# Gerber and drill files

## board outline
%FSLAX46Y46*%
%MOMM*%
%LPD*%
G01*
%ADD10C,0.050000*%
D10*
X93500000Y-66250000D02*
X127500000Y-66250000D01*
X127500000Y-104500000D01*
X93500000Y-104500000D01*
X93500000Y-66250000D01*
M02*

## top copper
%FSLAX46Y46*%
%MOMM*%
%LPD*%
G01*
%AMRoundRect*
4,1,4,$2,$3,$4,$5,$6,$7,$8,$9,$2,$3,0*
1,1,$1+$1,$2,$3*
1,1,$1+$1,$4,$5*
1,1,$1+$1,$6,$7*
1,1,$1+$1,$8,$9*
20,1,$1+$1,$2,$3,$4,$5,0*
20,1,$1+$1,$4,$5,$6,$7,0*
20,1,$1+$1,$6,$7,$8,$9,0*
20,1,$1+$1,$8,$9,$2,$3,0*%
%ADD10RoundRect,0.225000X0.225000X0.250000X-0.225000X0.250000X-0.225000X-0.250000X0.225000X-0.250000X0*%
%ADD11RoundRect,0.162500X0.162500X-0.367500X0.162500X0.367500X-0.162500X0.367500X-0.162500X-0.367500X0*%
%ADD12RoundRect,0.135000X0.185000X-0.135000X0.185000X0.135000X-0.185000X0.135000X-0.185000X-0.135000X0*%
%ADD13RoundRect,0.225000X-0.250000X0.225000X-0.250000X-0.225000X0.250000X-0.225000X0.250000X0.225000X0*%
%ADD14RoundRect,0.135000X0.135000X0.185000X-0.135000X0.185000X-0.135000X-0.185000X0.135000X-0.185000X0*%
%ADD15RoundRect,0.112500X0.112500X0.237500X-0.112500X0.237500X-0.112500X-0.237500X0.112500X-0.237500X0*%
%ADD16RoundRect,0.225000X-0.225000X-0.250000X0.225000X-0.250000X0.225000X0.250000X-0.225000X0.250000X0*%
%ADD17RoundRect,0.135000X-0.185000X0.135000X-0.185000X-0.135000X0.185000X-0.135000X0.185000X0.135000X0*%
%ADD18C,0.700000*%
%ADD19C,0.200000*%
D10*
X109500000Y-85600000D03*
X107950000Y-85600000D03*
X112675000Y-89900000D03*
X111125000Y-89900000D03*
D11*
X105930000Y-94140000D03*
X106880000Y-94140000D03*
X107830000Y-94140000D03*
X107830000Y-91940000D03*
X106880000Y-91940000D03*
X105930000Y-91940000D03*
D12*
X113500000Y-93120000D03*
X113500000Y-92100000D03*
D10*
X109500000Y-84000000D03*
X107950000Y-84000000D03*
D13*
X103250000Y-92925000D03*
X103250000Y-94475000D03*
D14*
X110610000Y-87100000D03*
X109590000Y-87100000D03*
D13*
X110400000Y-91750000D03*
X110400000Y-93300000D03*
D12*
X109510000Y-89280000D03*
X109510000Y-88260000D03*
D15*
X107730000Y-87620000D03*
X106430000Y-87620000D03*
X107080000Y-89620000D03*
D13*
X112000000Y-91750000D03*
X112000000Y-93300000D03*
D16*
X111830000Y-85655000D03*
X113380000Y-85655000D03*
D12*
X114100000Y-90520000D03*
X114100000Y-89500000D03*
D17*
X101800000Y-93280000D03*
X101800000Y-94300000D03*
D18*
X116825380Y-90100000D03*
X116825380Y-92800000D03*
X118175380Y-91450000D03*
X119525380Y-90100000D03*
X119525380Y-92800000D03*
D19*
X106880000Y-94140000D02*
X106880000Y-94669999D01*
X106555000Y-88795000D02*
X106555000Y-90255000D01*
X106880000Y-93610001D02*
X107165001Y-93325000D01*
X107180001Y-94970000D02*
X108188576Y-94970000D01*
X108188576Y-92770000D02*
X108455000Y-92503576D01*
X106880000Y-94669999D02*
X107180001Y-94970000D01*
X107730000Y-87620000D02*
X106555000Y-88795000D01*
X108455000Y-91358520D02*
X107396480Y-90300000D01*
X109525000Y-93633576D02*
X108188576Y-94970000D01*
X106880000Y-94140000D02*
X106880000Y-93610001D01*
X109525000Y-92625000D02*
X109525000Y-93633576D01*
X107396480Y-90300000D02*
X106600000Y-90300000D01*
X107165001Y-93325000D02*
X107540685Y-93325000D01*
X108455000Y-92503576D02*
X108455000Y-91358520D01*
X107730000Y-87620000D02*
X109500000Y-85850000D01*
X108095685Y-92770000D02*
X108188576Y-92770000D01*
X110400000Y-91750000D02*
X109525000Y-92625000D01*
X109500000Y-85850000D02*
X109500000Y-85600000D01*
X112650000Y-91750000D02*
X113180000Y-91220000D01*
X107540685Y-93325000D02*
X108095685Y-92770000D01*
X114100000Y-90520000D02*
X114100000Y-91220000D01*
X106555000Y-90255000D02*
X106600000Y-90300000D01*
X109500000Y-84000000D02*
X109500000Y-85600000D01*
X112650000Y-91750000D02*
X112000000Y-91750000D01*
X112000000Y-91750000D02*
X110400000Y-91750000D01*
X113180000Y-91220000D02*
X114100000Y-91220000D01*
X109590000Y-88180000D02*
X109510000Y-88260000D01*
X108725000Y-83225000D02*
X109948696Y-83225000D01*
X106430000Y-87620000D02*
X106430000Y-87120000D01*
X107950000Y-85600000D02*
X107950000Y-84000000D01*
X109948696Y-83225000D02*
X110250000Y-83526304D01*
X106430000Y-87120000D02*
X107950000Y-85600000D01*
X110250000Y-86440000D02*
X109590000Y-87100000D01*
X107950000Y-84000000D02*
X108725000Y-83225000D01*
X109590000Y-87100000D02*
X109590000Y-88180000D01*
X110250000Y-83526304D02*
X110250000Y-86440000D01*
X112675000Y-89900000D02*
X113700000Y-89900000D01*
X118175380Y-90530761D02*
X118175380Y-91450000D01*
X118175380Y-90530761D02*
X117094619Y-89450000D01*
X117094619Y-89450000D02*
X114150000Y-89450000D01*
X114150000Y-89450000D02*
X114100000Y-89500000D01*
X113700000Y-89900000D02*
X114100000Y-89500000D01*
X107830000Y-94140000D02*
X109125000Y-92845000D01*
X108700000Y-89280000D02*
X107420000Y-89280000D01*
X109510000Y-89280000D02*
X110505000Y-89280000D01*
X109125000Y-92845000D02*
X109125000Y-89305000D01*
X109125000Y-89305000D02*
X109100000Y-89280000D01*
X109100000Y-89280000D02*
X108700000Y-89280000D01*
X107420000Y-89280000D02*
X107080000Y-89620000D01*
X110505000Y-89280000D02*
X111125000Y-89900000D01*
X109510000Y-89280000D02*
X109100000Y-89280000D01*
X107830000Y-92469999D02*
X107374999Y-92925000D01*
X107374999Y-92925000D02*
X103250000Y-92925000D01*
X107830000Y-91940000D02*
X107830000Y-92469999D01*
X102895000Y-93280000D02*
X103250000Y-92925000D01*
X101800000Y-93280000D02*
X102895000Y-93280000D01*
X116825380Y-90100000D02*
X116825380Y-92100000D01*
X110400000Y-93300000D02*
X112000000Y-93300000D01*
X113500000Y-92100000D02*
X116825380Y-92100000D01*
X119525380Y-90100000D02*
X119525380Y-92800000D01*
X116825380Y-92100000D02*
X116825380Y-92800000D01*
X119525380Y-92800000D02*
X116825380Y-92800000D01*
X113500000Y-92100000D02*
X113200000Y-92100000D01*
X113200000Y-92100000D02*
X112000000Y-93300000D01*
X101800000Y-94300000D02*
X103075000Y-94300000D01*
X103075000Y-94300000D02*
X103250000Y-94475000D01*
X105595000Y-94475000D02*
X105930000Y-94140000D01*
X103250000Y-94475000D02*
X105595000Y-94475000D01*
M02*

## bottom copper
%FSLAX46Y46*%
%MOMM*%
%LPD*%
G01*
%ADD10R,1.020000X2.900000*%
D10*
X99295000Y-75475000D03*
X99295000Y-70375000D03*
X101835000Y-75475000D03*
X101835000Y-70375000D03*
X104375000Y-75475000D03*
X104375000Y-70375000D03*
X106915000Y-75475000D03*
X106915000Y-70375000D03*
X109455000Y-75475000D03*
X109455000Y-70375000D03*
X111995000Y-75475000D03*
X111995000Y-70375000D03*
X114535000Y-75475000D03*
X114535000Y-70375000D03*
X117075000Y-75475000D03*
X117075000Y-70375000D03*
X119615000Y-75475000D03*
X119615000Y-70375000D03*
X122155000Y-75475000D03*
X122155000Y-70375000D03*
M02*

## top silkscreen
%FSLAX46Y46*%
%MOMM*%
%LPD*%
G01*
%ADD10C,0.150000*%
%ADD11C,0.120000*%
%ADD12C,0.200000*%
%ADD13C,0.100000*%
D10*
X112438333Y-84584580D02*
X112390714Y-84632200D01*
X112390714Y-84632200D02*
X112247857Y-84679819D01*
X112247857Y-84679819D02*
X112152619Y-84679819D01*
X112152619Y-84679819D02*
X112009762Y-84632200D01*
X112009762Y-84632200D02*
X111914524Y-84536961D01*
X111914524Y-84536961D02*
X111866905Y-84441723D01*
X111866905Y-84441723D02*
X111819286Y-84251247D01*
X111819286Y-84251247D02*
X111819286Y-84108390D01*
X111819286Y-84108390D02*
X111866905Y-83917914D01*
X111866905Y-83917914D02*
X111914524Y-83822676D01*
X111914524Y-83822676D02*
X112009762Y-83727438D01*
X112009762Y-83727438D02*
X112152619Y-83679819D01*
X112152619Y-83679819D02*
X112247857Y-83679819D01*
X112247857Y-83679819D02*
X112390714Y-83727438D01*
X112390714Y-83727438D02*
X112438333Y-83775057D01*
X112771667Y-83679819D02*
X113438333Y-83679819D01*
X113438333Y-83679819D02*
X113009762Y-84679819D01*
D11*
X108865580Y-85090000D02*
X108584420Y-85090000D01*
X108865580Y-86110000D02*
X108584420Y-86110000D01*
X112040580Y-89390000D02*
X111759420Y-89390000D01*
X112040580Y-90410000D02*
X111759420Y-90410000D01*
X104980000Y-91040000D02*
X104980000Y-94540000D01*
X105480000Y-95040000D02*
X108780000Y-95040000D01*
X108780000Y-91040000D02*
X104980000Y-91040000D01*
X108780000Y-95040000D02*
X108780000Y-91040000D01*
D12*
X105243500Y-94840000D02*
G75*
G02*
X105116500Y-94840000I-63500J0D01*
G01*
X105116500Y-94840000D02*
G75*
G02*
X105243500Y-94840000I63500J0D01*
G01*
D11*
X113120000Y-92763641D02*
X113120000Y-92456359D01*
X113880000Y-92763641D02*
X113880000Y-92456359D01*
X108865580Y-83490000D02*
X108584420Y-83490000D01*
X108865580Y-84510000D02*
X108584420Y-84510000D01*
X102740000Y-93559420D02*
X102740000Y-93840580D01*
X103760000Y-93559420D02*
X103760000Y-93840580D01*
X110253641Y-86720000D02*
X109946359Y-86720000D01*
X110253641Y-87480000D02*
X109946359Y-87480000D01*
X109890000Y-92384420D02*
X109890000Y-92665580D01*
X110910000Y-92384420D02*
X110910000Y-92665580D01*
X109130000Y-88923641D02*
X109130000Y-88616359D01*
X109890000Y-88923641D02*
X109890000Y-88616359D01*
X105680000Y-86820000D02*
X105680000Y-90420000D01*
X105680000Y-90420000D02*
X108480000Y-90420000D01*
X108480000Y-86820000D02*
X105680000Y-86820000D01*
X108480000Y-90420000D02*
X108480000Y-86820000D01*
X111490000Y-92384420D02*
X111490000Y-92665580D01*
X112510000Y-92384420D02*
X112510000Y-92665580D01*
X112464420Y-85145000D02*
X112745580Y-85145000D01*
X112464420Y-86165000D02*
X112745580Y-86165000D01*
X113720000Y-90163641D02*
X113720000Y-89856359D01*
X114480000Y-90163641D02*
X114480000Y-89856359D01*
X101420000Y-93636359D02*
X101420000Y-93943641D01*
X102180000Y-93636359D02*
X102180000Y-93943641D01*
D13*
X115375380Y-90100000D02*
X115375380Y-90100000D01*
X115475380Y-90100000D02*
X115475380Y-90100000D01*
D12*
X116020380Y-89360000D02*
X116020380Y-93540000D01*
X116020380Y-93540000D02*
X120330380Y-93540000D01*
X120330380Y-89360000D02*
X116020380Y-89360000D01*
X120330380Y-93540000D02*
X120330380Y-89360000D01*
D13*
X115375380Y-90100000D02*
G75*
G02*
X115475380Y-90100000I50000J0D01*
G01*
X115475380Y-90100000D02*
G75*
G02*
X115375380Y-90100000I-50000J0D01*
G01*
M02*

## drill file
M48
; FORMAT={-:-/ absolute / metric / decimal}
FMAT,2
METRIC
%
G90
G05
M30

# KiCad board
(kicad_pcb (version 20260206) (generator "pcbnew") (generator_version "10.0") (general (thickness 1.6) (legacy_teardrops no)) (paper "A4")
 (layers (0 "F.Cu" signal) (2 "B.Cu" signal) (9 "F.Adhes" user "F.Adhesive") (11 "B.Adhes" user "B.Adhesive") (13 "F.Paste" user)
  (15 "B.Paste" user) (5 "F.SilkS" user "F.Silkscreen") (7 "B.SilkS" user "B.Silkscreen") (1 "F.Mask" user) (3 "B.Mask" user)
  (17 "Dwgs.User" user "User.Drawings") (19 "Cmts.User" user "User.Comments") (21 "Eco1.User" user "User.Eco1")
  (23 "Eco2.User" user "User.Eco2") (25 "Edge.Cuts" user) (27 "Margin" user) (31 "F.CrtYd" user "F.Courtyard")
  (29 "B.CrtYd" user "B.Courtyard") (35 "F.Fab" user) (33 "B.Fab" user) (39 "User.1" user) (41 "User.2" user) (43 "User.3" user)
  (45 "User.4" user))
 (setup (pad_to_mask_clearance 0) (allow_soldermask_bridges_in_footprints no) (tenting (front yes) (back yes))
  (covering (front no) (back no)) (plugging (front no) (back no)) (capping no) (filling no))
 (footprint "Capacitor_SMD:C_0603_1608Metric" (layer "F.Cu") (at 108.725 85.6 180)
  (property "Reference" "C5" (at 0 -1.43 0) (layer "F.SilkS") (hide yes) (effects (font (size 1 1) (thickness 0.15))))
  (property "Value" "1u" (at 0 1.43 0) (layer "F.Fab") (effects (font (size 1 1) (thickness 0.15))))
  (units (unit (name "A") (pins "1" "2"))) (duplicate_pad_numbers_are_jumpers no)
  (fp_line (start -0.14058 0.51) (end 0.14058 0.51) (stroke (width 0.12) (type solid)) (layer "F.SilkS"))
  (fp_line (start -0.14058 -0.51) (end 0.14058 -0.51) (stroke (width 0.12) (type solid)) (layer "F.SilkS"))
  (pad "1" smd roundrect (at -0.775 0 180) (size 0.9 0.95) (layers "F.Cu" "F.Mask" "F.Paste") (roundrect_rratio 0.25) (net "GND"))
  (pad "2" smd roundrect (at 0.775 0 180) (size 0.9 0.95) (layers "F.Cu" "F.Mask" "F.Paste") (roundrect_rratio 0.25) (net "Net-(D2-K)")))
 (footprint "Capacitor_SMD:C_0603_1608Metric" (layer "F.Cu") (at 111.9 89.9 180)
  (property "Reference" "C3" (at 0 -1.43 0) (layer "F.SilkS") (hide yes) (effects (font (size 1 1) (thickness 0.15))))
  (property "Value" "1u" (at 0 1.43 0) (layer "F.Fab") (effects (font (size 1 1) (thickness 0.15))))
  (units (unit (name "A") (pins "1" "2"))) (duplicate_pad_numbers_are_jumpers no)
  (fp_line (start -0.14058 0.51) (end 0.14058 0.51) (stroke (width 0.12) (type solid)) (layer "F.SilkS"))
  (fp_line (start -0.14058 -0.51) (end 0.14058 -0.51) (stroke (width 0.12) (type solid)) (layer "F.SilkS"))
  (pad "1" smd roundrect (at -0.775 0 180) (size 0.9 0.95) (layers "F.Cu" "F.Mask" "F.Paste") (roundrect_rratio 0.25) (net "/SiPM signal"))
  (pad "2" smd roundrect (at 0.775 0 180) (size 0.9 0.95) (layers "F.Cu" "F.Mask" "F.Paste") (roundrect_rratio 0.25) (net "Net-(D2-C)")))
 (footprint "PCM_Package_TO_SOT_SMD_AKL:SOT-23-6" (layer "F.Cu") (at 106.88 93.04 90)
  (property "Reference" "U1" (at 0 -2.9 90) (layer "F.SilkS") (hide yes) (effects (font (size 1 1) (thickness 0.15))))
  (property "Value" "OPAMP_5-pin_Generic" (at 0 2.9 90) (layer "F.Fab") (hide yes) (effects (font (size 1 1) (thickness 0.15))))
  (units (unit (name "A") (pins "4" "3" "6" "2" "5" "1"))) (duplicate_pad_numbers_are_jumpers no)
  (fp_line (start 2 -1.9) (end -1.5 -1.9) (stroke (width 0.12) (type solid)) (layer "F.SilkS"))
  (fp_line (start -2 -1.4) (end -2 1.9) (stroke (width 0.12) (type solid)) (layer "F.SilkS"))
  (fp_line (start 2 1.9) (end 2 -1.9) (stroke (width 0.12) (type solid)) (layer "F.SilkS"))
  (fp_line (start -2 1.9) (end 2 1.9) (stroke (width 0.12) (type solid)) (layer "F.SilkS"))
  (fp_circle (center -1.8 -1.7) (end -1.7365 -1.7) (stroke (width 0.2) (type solid)) (fill no) (layer "F.SilkS"))
  (pad "1" smd roundrect (at -1.1 -0.95 90) (size 1.06 0.65) (layers "F.Cu" "F.Mask" "F.Paste") (roundrect_rratio 0.25)
   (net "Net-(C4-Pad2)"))
  (pad "2" smd roundrect (at -1.1 0 90) (size 1.06 0.65) (layers "F.Cu" "F.Mask" "F.Paste") (roundrect_rratio 0.25) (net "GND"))
  (pad "3" smd roundrect (at -1.1 0.95 90) (size 1.06 0.65) (layers "F.Cu" "F.Mask" "F.Paste") (roundrect_rratio 0.25) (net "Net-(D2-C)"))
  (pad "4" smd roundrect (at 1.1 0.95 90) (size 1.06 0.65) (layers "F.Cu" "F.Mask" "F.Paste") (roundrect_rratio 0.25) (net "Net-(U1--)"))
  (pad "5" smd roundrect (at 1.1 0 90) (size 1.06 0.65) (layers "F.Cu" "F.Mask" "F.Paste") (roundrect_rratio 0.25)
   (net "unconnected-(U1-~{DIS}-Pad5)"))
  (pad "6" smd roundrect (at 1.1 -0.95 90) (size 1.06 0.65) (layers "F.Cu" "F.Mask" "F.Paste") (roundrect_rratio 0.25) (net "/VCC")))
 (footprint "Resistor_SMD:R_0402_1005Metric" (layer "F.Cu") (at 113.5 92.61 90)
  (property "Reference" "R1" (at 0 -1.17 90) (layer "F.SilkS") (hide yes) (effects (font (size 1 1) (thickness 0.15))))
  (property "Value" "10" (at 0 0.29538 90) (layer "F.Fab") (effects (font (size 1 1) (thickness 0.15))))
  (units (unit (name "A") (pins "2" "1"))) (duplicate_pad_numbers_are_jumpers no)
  (fp_line (start -0.153641 -0.38) (end 0.153641 -0.38) (stroke (width 0.12) (type solid)) (layer "F.SilkS"))
  (fp_line (start -0.153641 0.38) (end 0.153641 0.38) (stroke (width 0.12) (type solid)) (layer "F.SilkS"))
  (pad "1" smd roundrect (at -0.51 0 90) (size 0.54 0.64) (layers "F.Cu" "F.Mask" "F.Paste") (roundrect_rratio 0.25)
   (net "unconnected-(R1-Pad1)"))
  (pad "2" smd roundrect (at 0.51 0 90) (size 0.54 0.64) (layers "F.Cu" "F.Mask" "F.Paste") (roundrect_rratio 0.25) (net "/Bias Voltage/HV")))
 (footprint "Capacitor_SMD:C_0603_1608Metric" (layer "F.Cu") (at 108.725 84 180)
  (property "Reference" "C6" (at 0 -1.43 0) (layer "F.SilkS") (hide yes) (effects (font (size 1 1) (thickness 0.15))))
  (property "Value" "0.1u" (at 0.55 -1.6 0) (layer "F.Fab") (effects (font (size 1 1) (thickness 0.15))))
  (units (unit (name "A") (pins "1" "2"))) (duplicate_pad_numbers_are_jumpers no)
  (fp_line (start -0.14058 0.51) (end 0.14058 0.51) (stroke (width 0.12) (type solid)) (layer "F.SilkS"))
  (fp_line (start -0.14058 -0.51) (end 0.14058 -0.51) (stroke (width 0.12) (type solid)) (layer "F.SilkS"))
  (pad "1" smd roundrect (at -0.775 0 180) (size 0.9 0.95) (layers "F.Cu" "F.Mask" "F.Paste") (roundrect_rratio 0.25) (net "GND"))
  (pad "2" smd roundrect (at 0.775 0 180) (size 0.9 0.95) (layers "F.Cu" "F.Mask" "F.Paste") (roundrect_rratio 0.25) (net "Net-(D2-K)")))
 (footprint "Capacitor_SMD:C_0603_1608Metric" (layer "F.Cu") (at 103.25 93.7 -90)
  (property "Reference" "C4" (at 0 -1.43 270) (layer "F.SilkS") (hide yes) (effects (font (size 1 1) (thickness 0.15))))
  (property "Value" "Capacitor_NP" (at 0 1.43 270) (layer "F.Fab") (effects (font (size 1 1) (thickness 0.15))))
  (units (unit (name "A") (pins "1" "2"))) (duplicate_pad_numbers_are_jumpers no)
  (fp_line (start -0.14058 0.51) (end 0.14058 0.51) (stroke (width 0.12) (type solid)) (layer "F.SilkS"))
  (fp_line (start -0.14058 -0.51) (end 0.14058 -0.51) (stroke (width 0.12) (type solid)) (layer "F.SilkS"))
  (pad "1" smd roundrect (at -0.775 0 270) (size 0.9 0.95) (layers "F.Cu" "F.Mask" "F.Paste") (roundrect_rratio 0.25) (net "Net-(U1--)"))
  (pad "2" smd roundrect (at 0.775 0 270) (size 0.9 0.95) (layers "F.Cu" "F.Mask" "F.Paste") (roundrect_rratio 0.25) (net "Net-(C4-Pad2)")))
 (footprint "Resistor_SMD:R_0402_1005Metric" (layer "F.Cu") (at 110.1 87.1 180)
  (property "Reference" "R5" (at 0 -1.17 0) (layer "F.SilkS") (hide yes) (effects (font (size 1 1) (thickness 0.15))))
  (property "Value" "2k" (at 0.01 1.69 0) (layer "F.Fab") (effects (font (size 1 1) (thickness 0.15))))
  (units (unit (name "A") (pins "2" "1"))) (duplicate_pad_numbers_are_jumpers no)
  (fp_line (start -0.153641 0.38) (end 0.153641 0.38) (stroke (width 0.12) (type solid)) (layer "F.SilkS"))
  (fp_line (start -0.153641 -0.38) (end 0.153641 -0.38) (stroke (width 0.12) (type solid)) (layer "F.SilkS"))
  (pad "1" smd roundrect (at -0.51 0 180) (size 0.54 0.64) (layers "F.Cu" "F.Mask" "F.Paste") (roundrect_rratio 0.25) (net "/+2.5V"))
  (pad "2" smd roundrect (at 0.51 0 180) (size 0.54 0.64) (layers "F.Cu" "F.Mask" "F.Paste") (roundrect_rratio 0.25) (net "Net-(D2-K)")))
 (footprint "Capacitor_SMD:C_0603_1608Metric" (layer "F.Cu") (at 110.4 92.525 -90)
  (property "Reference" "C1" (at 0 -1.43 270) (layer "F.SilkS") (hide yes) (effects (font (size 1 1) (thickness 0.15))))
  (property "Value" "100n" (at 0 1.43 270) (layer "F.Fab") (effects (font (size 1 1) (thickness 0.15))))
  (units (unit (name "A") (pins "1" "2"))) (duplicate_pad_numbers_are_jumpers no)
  (fp_line (start -0.14058 0.51) (end 0.14058 0.51) (stroke (width 0.12) (type solid)) (layer "F.SilkS"))
  (fp_line (start -0.14058 -0.51) (end 0.14058 -0.51) (stroke (width 0.12) (type solid)) (layer "F.SilkS"))
  (pad "1" smd roundrect (at -0.775 0 270) (size 0.9 0.95) (layers "F.Cu" "F.Mask" "F.Paste") (roundrect_rratio 0.25) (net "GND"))
  (pad "2" smd roundrect (at 0.775 0 270) (size 0.9 0.95) (layers "F.Cu" "F.Mask" "F.Paste") (roundrect_rratio 0.25)
   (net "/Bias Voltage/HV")))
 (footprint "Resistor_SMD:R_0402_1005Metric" (layer "F.Cu") (at 109.51 88.77 90)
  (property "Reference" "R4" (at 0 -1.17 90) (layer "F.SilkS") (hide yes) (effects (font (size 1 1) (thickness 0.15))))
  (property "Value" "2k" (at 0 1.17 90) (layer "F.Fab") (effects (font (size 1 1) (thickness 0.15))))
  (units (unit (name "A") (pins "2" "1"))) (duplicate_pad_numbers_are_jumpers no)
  (fp_line (start -0.153641 -0.38) (end 0.153641 -0.38) (stroke (width 0.12) (type solid)) (layer "F.SilkS"))
  (fp_line (start -0.153641 0.38) (end 0.153641 0.38) (stroke (width 0.12) (type solid)) (layer "F.SilkS"))
  (pad "1" smd roundrect (at -0.51 0 90) (size 0.54 0.64) (layers "F.Cu" "F.Mask" "F.Paste") (roundrect_rratio 0.25) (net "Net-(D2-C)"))
  (pad "2" smd roundrect (at 0.51 0 90) (size 0.54 0.64) (layers "F.Cu" "F.Mask" "F.Paste") (roundrect_rratio 0.25) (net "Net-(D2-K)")))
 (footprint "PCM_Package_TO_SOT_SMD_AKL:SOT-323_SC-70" (layer "F.Cu") (at 107.08 88.62 -90)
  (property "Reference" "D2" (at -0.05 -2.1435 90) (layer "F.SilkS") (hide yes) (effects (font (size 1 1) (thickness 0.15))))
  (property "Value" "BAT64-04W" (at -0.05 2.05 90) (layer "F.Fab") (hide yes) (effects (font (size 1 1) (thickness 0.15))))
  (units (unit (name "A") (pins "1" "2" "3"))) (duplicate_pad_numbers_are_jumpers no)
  (fp_line (start -1.8 1.4) (end 1.8 1.4) (stroke (width 0.12) (type solid)) (layer "F.SilkS"))
  (fp_line (start 1.8 1.4) (end 1.8 -1.4) (stroke (width 0.12) (type solid)) (layer "F.SilkS"))
  (fp_line (start -1.8 -1.4) (end -1.8 1.4) (stroke (width 0.12) (type solid)) (layer "F.SilkS"))
  (fp_line (start 1.8 -1.4) (end -1.8 -1.4) (stroke (width 0.12) (type solid)) (layer "F.SilkS"))
  (pad "1" smd roundrect (at -1 -0.65 180) (size 0.45 0.7) (layers "F.Cu" "F.Mask" "F.Paste") (roundrect_rratio 0.25) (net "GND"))
  (pad "2" smd roundrect (at -1 0.65 180) (size 0.45 0.7) (layers "F.Cu" "F.Mask" "F.Paste") (roundrect_rratio 0.25) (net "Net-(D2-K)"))
  (pad "3" smd roundrect (at 1 0 180) (size 0.45 0.7) (layers "F.Cu" "F.Mask" "F.Paste") (roundrect_rratio 0.25) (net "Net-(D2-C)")))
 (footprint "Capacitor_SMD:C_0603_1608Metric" (layer "F.Cu") (at 112 92.525 -90)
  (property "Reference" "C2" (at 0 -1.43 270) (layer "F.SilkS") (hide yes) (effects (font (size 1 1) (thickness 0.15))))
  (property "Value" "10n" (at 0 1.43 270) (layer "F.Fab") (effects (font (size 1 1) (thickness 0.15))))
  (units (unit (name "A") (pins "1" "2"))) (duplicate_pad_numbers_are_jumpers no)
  (fp_line (start -0.14058 0.51) (end 0.14058 0.51) (stroke (width 0.12) (type solid)) (layer "F.SilkS"))
  (fp_line (start -0.14058 -0.51) (end 0.14058 -0.51) (stroke (width 0.12) (type solid)) (layer "F.SilkS"))
  (pad "1" smd roundrect (at -0.775 0 270) (size 0.9 0.95) (layers "F.Cu" "F.Mask" "F.Paste") (roundrect_rratio 0.25) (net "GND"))
  (pad "2" smd roundrect (at 0.775 0 270) (size 0.9 0.95) (layers "F.Cu" "F.Mask" "F.Paste") (roundrect_rratio 0.25)
   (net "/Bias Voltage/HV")))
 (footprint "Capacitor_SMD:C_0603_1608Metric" (layer "F.Cu") (at 112.605 85.655)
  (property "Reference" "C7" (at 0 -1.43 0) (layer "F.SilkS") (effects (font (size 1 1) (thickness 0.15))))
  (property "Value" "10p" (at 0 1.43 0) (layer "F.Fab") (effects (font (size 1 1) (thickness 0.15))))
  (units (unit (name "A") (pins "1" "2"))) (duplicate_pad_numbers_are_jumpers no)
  (fp_line (start -0.14058 -0.51) (end 0.14058 -0.51) (stroke (width 0.12) (type solid)) (layer "F.SilkS"))
  (fp_line (start -0.14058 0.51) (end 0.14058 0.51) (stroke (width 0.12) (type solid)) (layer "F.SilkS"))
  (pad "1" smd roundrect (at -0.775 0) (size 0.9 0.95) (layers "F.Cu" "F.Mask" "F.Paste") (roundrect_rratio 0.25) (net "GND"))
  (pad "2" smd roundrect (at 0.775 0) (size 0.9 0.95) (layers "F.Cu" "F.Mask" "F.Paste") (roundrect_rratio 0.25) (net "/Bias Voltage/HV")))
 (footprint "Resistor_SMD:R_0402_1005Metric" (layer "F.Cu") (at 114.1 90.01 90)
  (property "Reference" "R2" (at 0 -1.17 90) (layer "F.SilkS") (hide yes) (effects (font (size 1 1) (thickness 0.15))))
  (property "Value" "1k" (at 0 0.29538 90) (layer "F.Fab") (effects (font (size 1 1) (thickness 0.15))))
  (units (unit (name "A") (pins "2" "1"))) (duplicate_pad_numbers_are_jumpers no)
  (fp_line (start -0.153641 -0.38) (end 0.153641 -0.38) (stroke (width 0.12) (type solid)) (layer "F.SilkS"))
  (fp_line (start -0.153641 0.38) (end 0.153641 0.38) (stroke (width 0.12) (type solid)) (layer "F.SilkS"))
  (pad "1" smd roundrect (at -0.51 0 90) (size 0.54 0.64) (layers "F.Cu" "F.Mask" "F.Paste") (roundrect_rratio 0.25) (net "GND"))
  (pad "2" smd roundrect (at 0.51 0 90) (size 0.54 0.64) (layers "F.Cu" "F.Mask" "F.Paste") (roundrect_rratio 0.25) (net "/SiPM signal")))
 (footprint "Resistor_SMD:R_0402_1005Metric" (layer "F.Cu") (at 101.8 93.79 -90)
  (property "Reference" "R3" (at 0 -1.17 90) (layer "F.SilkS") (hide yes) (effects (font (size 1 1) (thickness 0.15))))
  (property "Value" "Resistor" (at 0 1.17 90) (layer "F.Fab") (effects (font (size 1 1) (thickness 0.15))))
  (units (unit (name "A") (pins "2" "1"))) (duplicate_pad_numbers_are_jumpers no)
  (fp_line (start -0.153641 0.38) (end 0.153641 0.38) (stroke (width 0.12) (type solid)) (layer "F.SilkS"))
  (fp_line (start -0.153641 -0.38) (end 0.153641 -0.38) (stroke (width 0.12) (type solid)) (layer "F.SilkS"))
  (pad "1" smd roundrect (at -0.51 0 270) (size 0.54 0.64) (layers "F.Cu" "F.Mask" "F.Paste") (roundrect_rratio 0.25) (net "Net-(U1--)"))
  (pad "2" smd roundrect (at 0.51 0 270) (size 0.54 0.64) (layers "F.Cu" "F.Mask" "F.Paste") (roundrect_rratio 0.25) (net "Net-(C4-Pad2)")))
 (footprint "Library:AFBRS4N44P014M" (layer "F.Cu") (at 118.17538 91.45 180)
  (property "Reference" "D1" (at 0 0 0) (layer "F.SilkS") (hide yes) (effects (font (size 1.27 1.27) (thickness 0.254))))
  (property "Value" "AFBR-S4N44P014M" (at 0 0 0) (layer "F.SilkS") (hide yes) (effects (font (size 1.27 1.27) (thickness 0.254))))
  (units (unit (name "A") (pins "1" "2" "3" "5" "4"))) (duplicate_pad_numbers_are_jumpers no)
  (fp_line (start 2.8 1.35) (end 2.8 1.35) (stroke (width 0.1) (type solid)) (layer "F.SilkS"))
  (fp_line (start 2.7 1.35) (end 2.7 1.35) (stroke (width 0.1) (type solid)) (layer "F.SilkS"))
  (fp_line (start 2.155 2.09) (end 2.155 -2.09) (stroke (width 0.2) (type solid)) (layer "F.SilkS"))
  (fp_line (start 2.155 -2.09) (end -2.155 -2.09) (stroke (width 0.2) (type solid)) (layer "F.SilkS"))
  (fp_line (start -2.155 2.09) (end 2.155 2.09) (stroke (width 0.2) (type solid)) (layer "F.SilkS"))
  (fp_line (start -2.155 -2.09) (end -2.155 2.09) (stroke (width 0.2) (type solid)) (layer "F.SilkS"))
  (fp_arc (start 2.8 1.35) (mid 2.75 1.4) (end 2.7 1.35) (stroke (width 0.1) (type solid)) (layer "F.SilkS"))
  (fp_arc (start 2.7 1.35) (mid 2.75 1.3) (end 2.8 1.35) (stroke (width 0.1) (type solid)) (layer "F.SilkS"))
  (pad "A1" smd circle (at 1.35 1.35 270) (size 0.7 0.7) (layers "F.Cu" "F.Mask" "F.Paste"))
  (pad "A3" smd circle (at 1.35 -1.35 270) (size 0.7 0.7) (layers "F.Cu" "F.Mask" "F.Paste"))
  (pad "B2" smd circle (at 0 0 270) (size 0.7 0.7) (layers "F.Cu" "F.Mask" "F.Paste"))
  (pad "C1" smd circle (at -1.35 1.35 270) (size 0.7 0.7) (layers "F.Cu" "F.Mask" "F.Paste"))
  (pad "C3" smd circle (at -1.35 -1.35 270) (size 0.7 0.7) (layers "F.Cu" "F.Mask" "F.Paste")))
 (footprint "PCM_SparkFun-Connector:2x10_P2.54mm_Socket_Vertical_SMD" (layer "B.Cu") (at 110.725 72.925 -90)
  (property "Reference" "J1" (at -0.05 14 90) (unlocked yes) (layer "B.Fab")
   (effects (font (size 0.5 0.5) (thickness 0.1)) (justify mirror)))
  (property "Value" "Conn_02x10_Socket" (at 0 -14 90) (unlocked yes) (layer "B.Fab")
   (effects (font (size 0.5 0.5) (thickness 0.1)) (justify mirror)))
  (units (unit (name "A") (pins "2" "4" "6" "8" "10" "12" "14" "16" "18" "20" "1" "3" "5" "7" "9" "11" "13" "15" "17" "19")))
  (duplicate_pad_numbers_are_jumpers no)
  (pad "1" smd rect (at 2.55 11.43 270) (size 2.9 1.02) (layers "B.Cu" "B.Mask" "B.Paste") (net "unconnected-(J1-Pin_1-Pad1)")
   (thermal_bridge_angle 0))
  (pad "2" smd rect (at -2.55 11.43 270) (size 2.9 1.02) (layers "B.Cu" "B.Mask" "B.Paste") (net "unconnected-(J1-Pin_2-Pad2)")
   (thermal_bridge_angle 0))
  (pad "3" smd rect (at 2.55 8.89 270) (size 2.9 1.02) (layers "B.Cu" "B.Mask" "B.Paste") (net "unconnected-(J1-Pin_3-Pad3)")
   (thermal_bridge_angle 0))
  (pad "4" smd rect (at -2.55 8.89 270) (size 2.9 1.02) (layers "B.Cu" "B.Mask" "B.Paste") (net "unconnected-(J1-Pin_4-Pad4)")
   (thermal_bridge_angle 0))
  (pad "5" smd rect (at 2.55 6.35 270) (size 2.9 1.02) (layers "B.Cu" "B.Mask" "B.Paste") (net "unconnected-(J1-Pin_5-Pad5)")
   (thermal_bridge_angle 0))
  (pad "6" smd rect (at -2.55 6.35 270) (size 2.9 1.02) (layers "B.Cu" "B.Mask" "B.Paste") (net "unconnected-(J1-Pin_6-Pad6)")
   (thermal_bridge_angle 0))
  (pad "7" smd rect (at 2.55 3.81 270) (size 2.9 1.02) (layers "B.Cu" "B.Mask" "B.Paste") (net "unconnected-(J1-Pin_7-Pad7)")
   (thermal_bridge_angle 0))
  (pad "8" smd rect (at -2.55 3.81 270) (size 2.9 1.02) (layers "B.Cu" "B.Mask" "B.Paste") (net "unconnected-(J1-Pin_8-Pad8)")
   (thermal_bridge_angle 0))
  (pad "9" smd rect (at 2.55 1.27 270) (size 2.9 1.02) (layers "B.Cu" "B.Mask" "B.Paste") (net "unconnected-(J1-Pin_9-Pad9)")
   (thermal_bridge_angle 0))
  (pad "10" smd rect (at -2.55 1.27 270) (size 2.9 1.02) (layers "B.Cu" "B.Mask" "B.Paste") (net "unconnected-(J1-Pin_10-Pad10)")
   (thermal_bridge_angle 0))
  (pad "11" smd rect (at 2.55 -1.27 270) (size 2.9 1.02) (layers "B.Cu" "B.Mask" "B.Paste") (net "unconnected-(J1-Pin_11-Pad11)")
   (thermal_bridge_angle 0))
  (pad "12" smd rect (at -2.55 -1.27 270) (size 2.9 1.02) (layers "B.Cu" "B.Mask" "B.Paste") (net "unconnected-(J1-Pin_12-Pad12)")
   (thermal_bridge_angle 0))
  (pad "13" smd rect (at 2.55 -3.81 270) (size 2.9 1.02) (layers "B.Cu" "B.Mask" "B.Paste") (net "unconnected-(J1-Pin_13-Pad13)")
   (thermal_bridge_angle 0))
  (pad "14" smd rect (at -2.55 -3.81 270) (size 2.9 1.02) (layers "B.Cu" "B.Mask" "B.Paste") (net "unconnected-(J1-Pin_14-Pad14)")
   (thermal_bridge_angle 0))
  (pad "15" smd rect (at 2.55 -6.35 270) (size 2.9 1.02) (layers "B.Cu" "B.Mask" "B.Paste") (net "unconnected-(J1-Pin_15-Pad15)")
   (thermal_bridge_angle 0))
  (pad "16" smd rect (at -2.55 -6.35 270) (size 2.9 1.02) (layers "B.Cu" "B.Mask" "B.Paste") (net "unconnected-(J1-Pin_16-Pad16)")
   (thermal_bridge_angle 0))
  (pad "17" smd rect (at 2.55 -8.89 270) (size 2.9 1.02) (layers "B.Cu" "B.Mask" "B.Paste") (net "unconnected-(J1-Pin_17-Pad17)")
   (thermal_bridge_angle 0))
  (pad "18" smd rect (at -2.55 -8.89 270) (size 2.9 1.02) (layers "B.Cu" "B.Mask" "B.Paste") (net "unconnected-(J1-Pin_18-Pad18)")
   (thermal_bridge_angle 0))
  (pad "19" smd rect (at 2.55 -11.43 270) (size 2.9 1.02) (layers "B.Cu" "B.Mask" "B.Paste") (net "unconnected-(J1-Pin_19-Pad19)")
   (thermal_bridge_angle 0))
  (pad "20" smd rect (at -2.55 -11.43 270) (size 2.9 1.02) (layers "B.Cu" "B.Mask" "B.Paste") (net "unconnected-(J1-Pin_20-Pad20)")
   (thermal_bridge_angle 0)))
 (gr_rect (start 93.5 66.25) (end 127.5 104.5) (stroke (width 0.05) (type default)) (fill no) (layer "Edge.Cuts"))
 (segment (start 106.88 94.14) (end 106.88 94.669999) (width 0.2) (layer "F.Cu") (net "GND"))
 (segment (start 106.555 88.795) (end 106.555 90.255) (width 0.2) (layer "F.Cu") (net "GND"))
 (segment (start 106.88 93.610001) (end 107.165001 93.325) (width 0.2) (layer "F.Cu") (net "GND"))
 (segment (start 107.180001 94.97) (end 108.188576 94.97) (width 0.2) (layer "F.Cu") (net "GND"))
 (segment (start 108.188576 92.77) (end 108.455 92.503576) (width 0.2) (layer "F.Cu") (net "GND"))
 (segment (start 106.88 94.669999) (end 107.180001 94.97) (width 0.2) (layer "F.Cu") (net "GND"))
 (segment (start 107.73 87.62) (end 106.555 88.795) (width 0.2) (layer "F.Cu") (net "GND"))
 (segment (start 108.455 91.35852) (end 107.39648 90.3) (width 0.2) (layer "F.Cu") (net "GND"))
 (segment (start 109.525 93.633576) (end 108.188576 94.97) (width 0.2) (layer "F.Cu") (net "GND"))
 (segment (start 106.88 94.14) (end 106.88 93.610001) (width 0.2) (layer "F.Cu") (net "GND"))
 (segment (start 109.525 92.625) (end 109.525 93.633576) (width 0.2) (layer "F.Cu") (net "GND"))
 (segment (start 107.39648 90.3) (end 106.6 90.3) (width 0.2) (layer "F.Cu") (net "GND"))
 (segment (start 107.165001 93.325) (end 107.540685 93.325) (width 0.2) (layer "F.Cu") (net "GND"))
 (segment (start 108.455 92.503576) (end 108.455 91.35852) (width 0.2) (layer "F.Cu") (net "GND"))
 (segment (start 107.73 87.62) (end 109.5 85.85) (width 0.2) (layer "F.Cu") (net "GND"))
 (segment (start 108.095685 92.77) (end 108.188576 92.77) (width 0.2) (layer "F.Cu") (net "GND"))
 (segment (start 110.4 91.75) (end 109.525 92.625) (width 0.2) (layer "F.Cu") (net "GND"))
 (segment (start 109.5 85.85) (end 109.5 85.6) (width 0.2) (layer "F.Cu") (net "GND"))
 (segment (start 112.65 91.75) (end 113.18 91.22) (width 0.2) (layer "F.Cu") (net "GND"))
 (segment (start 107.540685 93.325) (end 108.095685 92.77) (width 0.2) (layer "F.Cu") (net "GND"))
 (segment (start 114.1 90.52) (end 114.1 91.22) (width 0.2) (layer "F.Cu") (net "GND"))
 (segment (start 106.555 90.255) (end 106.6 90.3) (width 0.2) (layer "F.Cu") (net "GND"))
 (segment (start 109.5 84) (end 109.5 85.6) (width 0.2) (layer "F.Cu") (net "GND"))
 (segment (start 112.65 91.75) (end 112 91.75) (width 0.2) (layer "F.Cu") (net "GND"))
 (segment (start 112 91.75) (end 110.4 91.75) (width 0.2) (layer "F.Cu") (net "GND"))
 (segment (start 113.18 91.22) (end 114.1 91.22) (width 0.2) (layer "F.Cu") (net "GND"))
 (segment (start 109.59 88.18) (end 109.51 88.26) (width 0.2) (layer "F.Cu") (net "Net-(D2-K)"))
 (segment (start 108.725 83.225) (end 109.948696 83.225) (width 0.2) (layer "F.Cu") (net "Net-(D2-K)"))
 (segment (start 106.43 87.62) (end 106.43 87.12) (width 0.2) (layer "F.Cu") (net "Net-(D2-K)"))
 (segment (start 107.95 85.6) (end 107.95 84) (width 0.2) (layer "F.Cu") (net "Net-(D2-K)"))
 (segment (start 109.948696 83.225) (end 110.25 83.526304) (width 0.2) (layer "F.Cu") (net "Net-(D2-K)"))
 (segment (start 106.43 87.12) (end 107.95 85.6) (width 0.2) (layer "F.Cu") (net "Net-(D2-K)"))
 (segment (start 110.25 86.44) (end 109.59 87.1) (width 0.2) (layer "F.Cu") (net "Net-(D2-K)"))
 (segment (start 107.95 84) (end 108.725 83.225) (width 0.2) (layer "F.Cu") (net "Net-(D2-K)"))
 (segment (start 109.59 87.1) (end 109.59 88.18) (width 0.2) (layer "F.Cu") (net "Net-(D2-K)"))
 (segment (start 110.25 83.526304) (end 110.25 86.44) (width 0.2) (layer "F.Cu") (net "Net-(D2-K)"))
 (segment (start 112.675 89.9) (end 113.7 89.9) (width 0.2) (layer "F.Cu") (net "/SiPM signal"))
 (segment (start 118.17538 90.530761) (end 118.17538 91.45) (width 0.2) (layer "F.Cu") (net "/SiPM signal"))
 (segment (start 118.17538 90.530761) (end 117.094619 89.45) (width 0.2) (layer "F.Cu") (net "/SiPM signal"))
 (segment (start 117.094619 89.45) (end 114.15 89.45) (width 0.2) (layer "F.Cu") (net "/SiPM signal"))
 (segment (start 114.15 89.45) (end 114.1 89.5) (width 0.2) (layer "F.Cu") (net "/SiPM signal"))
 (segment (start 113.7 89.9) (end 114.1 89.5) (width 0.2) (layer "F.Cu") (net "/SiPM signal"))
 (segment (start 107.83 94.14) (end 109.125 92.845) (width 0.2) (layer "F.Cu") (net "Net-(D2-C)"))
 (segment (start 108.7 89.28) (end 107.42 89.28) (width 0.2) (layer "F.Cu") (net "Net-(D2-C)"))
 (segment (start 109.51 89.28) (end 110.505 89.28) (width 0.2) (layer "F.Cu") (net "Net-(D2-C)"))
 (segment (start 109.125 92.845) (end 109.125 89.305) (width 0.2) (layer "F.Cu") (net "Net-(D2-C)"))
 (segment (start 109.125 89.305) (end 109.1 89.28) (width 0.2) (layer "F.Cu") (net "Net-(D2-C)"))
 (segment (start 109.1 89.28) (end 108.7 89.28) (width 0.2) (layer "F.Cu") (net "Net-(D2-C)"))
 (segment (start 107.42 89.28) (end 107.08 89.62) (width 0.2) (layer "F.Cu") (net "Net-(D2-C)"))
 (segment (start 110.505 89.28) (end 111.125 89.9) (width 0.2) (layer "F.Cu") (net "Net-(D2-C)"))
 (segment (start 109.51 89.28) (end 109.1 89.28) (width 0.2) (layer "F.Cu") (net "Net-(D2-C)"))
 (segment (start 107.83 92.469999) (end 107.374999 92.925) (width 0.2) (layer "F.Cu") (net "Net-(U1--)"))
 (segment (start 107.374999 92.925) (end 103.25 92.925) (width 0.2) (layer "F.Cu") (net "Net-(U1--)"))
 (segment (start 107.83 91.94) (end 107.83 92.469999) (width 0.2) (layer "F.Cu") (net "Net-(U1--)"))
 (segment (start 102.895 93.28) (end 103.25 92.925) (width 0.2) (layer "F.Cu") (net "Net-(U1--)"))
 (segment (start 101.8 93.28) (end 102.895 93.28) (width 0.2) (layer "F.Cu") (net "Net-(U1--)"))
 (segment (start 116.82538 90.1) (end 116.82538 92.1) (width 0.2) (layer "F.Cu") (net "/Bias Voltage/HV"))
 (segment (start 110.4 93.3) (end 112 93.3) (width 0.2) (layer "F.Cu") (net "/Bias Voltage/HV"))
 (segment (start 113.5 92.1) (end 116.82538 92.1) (width 0.2) (layer "F.Cu") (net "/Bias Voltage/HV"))
 (segment (start 119.52538 90.1) (end 119.52538 92.8) (width 0.2) (layer "F.Cu") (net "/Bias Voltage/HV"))
 (segment (start 116.82538 92.1) (end 116.82538 92.8) (width 0.2) (layer "F.Cu") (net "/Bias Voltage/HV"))
 (segment (start 119.52538 92.8) (end 116.82538 92.8) (width 0.2) (layer "F.Cu") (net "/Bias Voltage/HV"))
 (segment (start 113.5 92.1) (end 113.2 92.1) (width 0.2) (layer "F.Cu") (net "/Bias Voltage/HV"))
 (segment (start 113.2 92.1) (end 112 93.3) (width 0.2) (layer "F.Cu") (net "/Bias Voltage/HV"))
 (segment (start 101.8 94.3) (end 103.075 94.3) (width 0.2) (layer "F.Cu") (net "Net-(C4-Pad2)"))
 (segment (start 103.075 94.3) (end 103.25 94.475) (width 0.2) (layer "F.Cu") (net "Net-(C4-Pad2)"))
 (segment (start 105.595 94.475) (end 105.93 94.14) (width 0.2) (layer "F.Cu") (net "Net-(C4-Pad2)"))
 (segment (start 103.25 94.475) (end 105.595 94.475) (width 0.2) (layer "F.Cu") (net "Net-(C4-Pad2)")))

